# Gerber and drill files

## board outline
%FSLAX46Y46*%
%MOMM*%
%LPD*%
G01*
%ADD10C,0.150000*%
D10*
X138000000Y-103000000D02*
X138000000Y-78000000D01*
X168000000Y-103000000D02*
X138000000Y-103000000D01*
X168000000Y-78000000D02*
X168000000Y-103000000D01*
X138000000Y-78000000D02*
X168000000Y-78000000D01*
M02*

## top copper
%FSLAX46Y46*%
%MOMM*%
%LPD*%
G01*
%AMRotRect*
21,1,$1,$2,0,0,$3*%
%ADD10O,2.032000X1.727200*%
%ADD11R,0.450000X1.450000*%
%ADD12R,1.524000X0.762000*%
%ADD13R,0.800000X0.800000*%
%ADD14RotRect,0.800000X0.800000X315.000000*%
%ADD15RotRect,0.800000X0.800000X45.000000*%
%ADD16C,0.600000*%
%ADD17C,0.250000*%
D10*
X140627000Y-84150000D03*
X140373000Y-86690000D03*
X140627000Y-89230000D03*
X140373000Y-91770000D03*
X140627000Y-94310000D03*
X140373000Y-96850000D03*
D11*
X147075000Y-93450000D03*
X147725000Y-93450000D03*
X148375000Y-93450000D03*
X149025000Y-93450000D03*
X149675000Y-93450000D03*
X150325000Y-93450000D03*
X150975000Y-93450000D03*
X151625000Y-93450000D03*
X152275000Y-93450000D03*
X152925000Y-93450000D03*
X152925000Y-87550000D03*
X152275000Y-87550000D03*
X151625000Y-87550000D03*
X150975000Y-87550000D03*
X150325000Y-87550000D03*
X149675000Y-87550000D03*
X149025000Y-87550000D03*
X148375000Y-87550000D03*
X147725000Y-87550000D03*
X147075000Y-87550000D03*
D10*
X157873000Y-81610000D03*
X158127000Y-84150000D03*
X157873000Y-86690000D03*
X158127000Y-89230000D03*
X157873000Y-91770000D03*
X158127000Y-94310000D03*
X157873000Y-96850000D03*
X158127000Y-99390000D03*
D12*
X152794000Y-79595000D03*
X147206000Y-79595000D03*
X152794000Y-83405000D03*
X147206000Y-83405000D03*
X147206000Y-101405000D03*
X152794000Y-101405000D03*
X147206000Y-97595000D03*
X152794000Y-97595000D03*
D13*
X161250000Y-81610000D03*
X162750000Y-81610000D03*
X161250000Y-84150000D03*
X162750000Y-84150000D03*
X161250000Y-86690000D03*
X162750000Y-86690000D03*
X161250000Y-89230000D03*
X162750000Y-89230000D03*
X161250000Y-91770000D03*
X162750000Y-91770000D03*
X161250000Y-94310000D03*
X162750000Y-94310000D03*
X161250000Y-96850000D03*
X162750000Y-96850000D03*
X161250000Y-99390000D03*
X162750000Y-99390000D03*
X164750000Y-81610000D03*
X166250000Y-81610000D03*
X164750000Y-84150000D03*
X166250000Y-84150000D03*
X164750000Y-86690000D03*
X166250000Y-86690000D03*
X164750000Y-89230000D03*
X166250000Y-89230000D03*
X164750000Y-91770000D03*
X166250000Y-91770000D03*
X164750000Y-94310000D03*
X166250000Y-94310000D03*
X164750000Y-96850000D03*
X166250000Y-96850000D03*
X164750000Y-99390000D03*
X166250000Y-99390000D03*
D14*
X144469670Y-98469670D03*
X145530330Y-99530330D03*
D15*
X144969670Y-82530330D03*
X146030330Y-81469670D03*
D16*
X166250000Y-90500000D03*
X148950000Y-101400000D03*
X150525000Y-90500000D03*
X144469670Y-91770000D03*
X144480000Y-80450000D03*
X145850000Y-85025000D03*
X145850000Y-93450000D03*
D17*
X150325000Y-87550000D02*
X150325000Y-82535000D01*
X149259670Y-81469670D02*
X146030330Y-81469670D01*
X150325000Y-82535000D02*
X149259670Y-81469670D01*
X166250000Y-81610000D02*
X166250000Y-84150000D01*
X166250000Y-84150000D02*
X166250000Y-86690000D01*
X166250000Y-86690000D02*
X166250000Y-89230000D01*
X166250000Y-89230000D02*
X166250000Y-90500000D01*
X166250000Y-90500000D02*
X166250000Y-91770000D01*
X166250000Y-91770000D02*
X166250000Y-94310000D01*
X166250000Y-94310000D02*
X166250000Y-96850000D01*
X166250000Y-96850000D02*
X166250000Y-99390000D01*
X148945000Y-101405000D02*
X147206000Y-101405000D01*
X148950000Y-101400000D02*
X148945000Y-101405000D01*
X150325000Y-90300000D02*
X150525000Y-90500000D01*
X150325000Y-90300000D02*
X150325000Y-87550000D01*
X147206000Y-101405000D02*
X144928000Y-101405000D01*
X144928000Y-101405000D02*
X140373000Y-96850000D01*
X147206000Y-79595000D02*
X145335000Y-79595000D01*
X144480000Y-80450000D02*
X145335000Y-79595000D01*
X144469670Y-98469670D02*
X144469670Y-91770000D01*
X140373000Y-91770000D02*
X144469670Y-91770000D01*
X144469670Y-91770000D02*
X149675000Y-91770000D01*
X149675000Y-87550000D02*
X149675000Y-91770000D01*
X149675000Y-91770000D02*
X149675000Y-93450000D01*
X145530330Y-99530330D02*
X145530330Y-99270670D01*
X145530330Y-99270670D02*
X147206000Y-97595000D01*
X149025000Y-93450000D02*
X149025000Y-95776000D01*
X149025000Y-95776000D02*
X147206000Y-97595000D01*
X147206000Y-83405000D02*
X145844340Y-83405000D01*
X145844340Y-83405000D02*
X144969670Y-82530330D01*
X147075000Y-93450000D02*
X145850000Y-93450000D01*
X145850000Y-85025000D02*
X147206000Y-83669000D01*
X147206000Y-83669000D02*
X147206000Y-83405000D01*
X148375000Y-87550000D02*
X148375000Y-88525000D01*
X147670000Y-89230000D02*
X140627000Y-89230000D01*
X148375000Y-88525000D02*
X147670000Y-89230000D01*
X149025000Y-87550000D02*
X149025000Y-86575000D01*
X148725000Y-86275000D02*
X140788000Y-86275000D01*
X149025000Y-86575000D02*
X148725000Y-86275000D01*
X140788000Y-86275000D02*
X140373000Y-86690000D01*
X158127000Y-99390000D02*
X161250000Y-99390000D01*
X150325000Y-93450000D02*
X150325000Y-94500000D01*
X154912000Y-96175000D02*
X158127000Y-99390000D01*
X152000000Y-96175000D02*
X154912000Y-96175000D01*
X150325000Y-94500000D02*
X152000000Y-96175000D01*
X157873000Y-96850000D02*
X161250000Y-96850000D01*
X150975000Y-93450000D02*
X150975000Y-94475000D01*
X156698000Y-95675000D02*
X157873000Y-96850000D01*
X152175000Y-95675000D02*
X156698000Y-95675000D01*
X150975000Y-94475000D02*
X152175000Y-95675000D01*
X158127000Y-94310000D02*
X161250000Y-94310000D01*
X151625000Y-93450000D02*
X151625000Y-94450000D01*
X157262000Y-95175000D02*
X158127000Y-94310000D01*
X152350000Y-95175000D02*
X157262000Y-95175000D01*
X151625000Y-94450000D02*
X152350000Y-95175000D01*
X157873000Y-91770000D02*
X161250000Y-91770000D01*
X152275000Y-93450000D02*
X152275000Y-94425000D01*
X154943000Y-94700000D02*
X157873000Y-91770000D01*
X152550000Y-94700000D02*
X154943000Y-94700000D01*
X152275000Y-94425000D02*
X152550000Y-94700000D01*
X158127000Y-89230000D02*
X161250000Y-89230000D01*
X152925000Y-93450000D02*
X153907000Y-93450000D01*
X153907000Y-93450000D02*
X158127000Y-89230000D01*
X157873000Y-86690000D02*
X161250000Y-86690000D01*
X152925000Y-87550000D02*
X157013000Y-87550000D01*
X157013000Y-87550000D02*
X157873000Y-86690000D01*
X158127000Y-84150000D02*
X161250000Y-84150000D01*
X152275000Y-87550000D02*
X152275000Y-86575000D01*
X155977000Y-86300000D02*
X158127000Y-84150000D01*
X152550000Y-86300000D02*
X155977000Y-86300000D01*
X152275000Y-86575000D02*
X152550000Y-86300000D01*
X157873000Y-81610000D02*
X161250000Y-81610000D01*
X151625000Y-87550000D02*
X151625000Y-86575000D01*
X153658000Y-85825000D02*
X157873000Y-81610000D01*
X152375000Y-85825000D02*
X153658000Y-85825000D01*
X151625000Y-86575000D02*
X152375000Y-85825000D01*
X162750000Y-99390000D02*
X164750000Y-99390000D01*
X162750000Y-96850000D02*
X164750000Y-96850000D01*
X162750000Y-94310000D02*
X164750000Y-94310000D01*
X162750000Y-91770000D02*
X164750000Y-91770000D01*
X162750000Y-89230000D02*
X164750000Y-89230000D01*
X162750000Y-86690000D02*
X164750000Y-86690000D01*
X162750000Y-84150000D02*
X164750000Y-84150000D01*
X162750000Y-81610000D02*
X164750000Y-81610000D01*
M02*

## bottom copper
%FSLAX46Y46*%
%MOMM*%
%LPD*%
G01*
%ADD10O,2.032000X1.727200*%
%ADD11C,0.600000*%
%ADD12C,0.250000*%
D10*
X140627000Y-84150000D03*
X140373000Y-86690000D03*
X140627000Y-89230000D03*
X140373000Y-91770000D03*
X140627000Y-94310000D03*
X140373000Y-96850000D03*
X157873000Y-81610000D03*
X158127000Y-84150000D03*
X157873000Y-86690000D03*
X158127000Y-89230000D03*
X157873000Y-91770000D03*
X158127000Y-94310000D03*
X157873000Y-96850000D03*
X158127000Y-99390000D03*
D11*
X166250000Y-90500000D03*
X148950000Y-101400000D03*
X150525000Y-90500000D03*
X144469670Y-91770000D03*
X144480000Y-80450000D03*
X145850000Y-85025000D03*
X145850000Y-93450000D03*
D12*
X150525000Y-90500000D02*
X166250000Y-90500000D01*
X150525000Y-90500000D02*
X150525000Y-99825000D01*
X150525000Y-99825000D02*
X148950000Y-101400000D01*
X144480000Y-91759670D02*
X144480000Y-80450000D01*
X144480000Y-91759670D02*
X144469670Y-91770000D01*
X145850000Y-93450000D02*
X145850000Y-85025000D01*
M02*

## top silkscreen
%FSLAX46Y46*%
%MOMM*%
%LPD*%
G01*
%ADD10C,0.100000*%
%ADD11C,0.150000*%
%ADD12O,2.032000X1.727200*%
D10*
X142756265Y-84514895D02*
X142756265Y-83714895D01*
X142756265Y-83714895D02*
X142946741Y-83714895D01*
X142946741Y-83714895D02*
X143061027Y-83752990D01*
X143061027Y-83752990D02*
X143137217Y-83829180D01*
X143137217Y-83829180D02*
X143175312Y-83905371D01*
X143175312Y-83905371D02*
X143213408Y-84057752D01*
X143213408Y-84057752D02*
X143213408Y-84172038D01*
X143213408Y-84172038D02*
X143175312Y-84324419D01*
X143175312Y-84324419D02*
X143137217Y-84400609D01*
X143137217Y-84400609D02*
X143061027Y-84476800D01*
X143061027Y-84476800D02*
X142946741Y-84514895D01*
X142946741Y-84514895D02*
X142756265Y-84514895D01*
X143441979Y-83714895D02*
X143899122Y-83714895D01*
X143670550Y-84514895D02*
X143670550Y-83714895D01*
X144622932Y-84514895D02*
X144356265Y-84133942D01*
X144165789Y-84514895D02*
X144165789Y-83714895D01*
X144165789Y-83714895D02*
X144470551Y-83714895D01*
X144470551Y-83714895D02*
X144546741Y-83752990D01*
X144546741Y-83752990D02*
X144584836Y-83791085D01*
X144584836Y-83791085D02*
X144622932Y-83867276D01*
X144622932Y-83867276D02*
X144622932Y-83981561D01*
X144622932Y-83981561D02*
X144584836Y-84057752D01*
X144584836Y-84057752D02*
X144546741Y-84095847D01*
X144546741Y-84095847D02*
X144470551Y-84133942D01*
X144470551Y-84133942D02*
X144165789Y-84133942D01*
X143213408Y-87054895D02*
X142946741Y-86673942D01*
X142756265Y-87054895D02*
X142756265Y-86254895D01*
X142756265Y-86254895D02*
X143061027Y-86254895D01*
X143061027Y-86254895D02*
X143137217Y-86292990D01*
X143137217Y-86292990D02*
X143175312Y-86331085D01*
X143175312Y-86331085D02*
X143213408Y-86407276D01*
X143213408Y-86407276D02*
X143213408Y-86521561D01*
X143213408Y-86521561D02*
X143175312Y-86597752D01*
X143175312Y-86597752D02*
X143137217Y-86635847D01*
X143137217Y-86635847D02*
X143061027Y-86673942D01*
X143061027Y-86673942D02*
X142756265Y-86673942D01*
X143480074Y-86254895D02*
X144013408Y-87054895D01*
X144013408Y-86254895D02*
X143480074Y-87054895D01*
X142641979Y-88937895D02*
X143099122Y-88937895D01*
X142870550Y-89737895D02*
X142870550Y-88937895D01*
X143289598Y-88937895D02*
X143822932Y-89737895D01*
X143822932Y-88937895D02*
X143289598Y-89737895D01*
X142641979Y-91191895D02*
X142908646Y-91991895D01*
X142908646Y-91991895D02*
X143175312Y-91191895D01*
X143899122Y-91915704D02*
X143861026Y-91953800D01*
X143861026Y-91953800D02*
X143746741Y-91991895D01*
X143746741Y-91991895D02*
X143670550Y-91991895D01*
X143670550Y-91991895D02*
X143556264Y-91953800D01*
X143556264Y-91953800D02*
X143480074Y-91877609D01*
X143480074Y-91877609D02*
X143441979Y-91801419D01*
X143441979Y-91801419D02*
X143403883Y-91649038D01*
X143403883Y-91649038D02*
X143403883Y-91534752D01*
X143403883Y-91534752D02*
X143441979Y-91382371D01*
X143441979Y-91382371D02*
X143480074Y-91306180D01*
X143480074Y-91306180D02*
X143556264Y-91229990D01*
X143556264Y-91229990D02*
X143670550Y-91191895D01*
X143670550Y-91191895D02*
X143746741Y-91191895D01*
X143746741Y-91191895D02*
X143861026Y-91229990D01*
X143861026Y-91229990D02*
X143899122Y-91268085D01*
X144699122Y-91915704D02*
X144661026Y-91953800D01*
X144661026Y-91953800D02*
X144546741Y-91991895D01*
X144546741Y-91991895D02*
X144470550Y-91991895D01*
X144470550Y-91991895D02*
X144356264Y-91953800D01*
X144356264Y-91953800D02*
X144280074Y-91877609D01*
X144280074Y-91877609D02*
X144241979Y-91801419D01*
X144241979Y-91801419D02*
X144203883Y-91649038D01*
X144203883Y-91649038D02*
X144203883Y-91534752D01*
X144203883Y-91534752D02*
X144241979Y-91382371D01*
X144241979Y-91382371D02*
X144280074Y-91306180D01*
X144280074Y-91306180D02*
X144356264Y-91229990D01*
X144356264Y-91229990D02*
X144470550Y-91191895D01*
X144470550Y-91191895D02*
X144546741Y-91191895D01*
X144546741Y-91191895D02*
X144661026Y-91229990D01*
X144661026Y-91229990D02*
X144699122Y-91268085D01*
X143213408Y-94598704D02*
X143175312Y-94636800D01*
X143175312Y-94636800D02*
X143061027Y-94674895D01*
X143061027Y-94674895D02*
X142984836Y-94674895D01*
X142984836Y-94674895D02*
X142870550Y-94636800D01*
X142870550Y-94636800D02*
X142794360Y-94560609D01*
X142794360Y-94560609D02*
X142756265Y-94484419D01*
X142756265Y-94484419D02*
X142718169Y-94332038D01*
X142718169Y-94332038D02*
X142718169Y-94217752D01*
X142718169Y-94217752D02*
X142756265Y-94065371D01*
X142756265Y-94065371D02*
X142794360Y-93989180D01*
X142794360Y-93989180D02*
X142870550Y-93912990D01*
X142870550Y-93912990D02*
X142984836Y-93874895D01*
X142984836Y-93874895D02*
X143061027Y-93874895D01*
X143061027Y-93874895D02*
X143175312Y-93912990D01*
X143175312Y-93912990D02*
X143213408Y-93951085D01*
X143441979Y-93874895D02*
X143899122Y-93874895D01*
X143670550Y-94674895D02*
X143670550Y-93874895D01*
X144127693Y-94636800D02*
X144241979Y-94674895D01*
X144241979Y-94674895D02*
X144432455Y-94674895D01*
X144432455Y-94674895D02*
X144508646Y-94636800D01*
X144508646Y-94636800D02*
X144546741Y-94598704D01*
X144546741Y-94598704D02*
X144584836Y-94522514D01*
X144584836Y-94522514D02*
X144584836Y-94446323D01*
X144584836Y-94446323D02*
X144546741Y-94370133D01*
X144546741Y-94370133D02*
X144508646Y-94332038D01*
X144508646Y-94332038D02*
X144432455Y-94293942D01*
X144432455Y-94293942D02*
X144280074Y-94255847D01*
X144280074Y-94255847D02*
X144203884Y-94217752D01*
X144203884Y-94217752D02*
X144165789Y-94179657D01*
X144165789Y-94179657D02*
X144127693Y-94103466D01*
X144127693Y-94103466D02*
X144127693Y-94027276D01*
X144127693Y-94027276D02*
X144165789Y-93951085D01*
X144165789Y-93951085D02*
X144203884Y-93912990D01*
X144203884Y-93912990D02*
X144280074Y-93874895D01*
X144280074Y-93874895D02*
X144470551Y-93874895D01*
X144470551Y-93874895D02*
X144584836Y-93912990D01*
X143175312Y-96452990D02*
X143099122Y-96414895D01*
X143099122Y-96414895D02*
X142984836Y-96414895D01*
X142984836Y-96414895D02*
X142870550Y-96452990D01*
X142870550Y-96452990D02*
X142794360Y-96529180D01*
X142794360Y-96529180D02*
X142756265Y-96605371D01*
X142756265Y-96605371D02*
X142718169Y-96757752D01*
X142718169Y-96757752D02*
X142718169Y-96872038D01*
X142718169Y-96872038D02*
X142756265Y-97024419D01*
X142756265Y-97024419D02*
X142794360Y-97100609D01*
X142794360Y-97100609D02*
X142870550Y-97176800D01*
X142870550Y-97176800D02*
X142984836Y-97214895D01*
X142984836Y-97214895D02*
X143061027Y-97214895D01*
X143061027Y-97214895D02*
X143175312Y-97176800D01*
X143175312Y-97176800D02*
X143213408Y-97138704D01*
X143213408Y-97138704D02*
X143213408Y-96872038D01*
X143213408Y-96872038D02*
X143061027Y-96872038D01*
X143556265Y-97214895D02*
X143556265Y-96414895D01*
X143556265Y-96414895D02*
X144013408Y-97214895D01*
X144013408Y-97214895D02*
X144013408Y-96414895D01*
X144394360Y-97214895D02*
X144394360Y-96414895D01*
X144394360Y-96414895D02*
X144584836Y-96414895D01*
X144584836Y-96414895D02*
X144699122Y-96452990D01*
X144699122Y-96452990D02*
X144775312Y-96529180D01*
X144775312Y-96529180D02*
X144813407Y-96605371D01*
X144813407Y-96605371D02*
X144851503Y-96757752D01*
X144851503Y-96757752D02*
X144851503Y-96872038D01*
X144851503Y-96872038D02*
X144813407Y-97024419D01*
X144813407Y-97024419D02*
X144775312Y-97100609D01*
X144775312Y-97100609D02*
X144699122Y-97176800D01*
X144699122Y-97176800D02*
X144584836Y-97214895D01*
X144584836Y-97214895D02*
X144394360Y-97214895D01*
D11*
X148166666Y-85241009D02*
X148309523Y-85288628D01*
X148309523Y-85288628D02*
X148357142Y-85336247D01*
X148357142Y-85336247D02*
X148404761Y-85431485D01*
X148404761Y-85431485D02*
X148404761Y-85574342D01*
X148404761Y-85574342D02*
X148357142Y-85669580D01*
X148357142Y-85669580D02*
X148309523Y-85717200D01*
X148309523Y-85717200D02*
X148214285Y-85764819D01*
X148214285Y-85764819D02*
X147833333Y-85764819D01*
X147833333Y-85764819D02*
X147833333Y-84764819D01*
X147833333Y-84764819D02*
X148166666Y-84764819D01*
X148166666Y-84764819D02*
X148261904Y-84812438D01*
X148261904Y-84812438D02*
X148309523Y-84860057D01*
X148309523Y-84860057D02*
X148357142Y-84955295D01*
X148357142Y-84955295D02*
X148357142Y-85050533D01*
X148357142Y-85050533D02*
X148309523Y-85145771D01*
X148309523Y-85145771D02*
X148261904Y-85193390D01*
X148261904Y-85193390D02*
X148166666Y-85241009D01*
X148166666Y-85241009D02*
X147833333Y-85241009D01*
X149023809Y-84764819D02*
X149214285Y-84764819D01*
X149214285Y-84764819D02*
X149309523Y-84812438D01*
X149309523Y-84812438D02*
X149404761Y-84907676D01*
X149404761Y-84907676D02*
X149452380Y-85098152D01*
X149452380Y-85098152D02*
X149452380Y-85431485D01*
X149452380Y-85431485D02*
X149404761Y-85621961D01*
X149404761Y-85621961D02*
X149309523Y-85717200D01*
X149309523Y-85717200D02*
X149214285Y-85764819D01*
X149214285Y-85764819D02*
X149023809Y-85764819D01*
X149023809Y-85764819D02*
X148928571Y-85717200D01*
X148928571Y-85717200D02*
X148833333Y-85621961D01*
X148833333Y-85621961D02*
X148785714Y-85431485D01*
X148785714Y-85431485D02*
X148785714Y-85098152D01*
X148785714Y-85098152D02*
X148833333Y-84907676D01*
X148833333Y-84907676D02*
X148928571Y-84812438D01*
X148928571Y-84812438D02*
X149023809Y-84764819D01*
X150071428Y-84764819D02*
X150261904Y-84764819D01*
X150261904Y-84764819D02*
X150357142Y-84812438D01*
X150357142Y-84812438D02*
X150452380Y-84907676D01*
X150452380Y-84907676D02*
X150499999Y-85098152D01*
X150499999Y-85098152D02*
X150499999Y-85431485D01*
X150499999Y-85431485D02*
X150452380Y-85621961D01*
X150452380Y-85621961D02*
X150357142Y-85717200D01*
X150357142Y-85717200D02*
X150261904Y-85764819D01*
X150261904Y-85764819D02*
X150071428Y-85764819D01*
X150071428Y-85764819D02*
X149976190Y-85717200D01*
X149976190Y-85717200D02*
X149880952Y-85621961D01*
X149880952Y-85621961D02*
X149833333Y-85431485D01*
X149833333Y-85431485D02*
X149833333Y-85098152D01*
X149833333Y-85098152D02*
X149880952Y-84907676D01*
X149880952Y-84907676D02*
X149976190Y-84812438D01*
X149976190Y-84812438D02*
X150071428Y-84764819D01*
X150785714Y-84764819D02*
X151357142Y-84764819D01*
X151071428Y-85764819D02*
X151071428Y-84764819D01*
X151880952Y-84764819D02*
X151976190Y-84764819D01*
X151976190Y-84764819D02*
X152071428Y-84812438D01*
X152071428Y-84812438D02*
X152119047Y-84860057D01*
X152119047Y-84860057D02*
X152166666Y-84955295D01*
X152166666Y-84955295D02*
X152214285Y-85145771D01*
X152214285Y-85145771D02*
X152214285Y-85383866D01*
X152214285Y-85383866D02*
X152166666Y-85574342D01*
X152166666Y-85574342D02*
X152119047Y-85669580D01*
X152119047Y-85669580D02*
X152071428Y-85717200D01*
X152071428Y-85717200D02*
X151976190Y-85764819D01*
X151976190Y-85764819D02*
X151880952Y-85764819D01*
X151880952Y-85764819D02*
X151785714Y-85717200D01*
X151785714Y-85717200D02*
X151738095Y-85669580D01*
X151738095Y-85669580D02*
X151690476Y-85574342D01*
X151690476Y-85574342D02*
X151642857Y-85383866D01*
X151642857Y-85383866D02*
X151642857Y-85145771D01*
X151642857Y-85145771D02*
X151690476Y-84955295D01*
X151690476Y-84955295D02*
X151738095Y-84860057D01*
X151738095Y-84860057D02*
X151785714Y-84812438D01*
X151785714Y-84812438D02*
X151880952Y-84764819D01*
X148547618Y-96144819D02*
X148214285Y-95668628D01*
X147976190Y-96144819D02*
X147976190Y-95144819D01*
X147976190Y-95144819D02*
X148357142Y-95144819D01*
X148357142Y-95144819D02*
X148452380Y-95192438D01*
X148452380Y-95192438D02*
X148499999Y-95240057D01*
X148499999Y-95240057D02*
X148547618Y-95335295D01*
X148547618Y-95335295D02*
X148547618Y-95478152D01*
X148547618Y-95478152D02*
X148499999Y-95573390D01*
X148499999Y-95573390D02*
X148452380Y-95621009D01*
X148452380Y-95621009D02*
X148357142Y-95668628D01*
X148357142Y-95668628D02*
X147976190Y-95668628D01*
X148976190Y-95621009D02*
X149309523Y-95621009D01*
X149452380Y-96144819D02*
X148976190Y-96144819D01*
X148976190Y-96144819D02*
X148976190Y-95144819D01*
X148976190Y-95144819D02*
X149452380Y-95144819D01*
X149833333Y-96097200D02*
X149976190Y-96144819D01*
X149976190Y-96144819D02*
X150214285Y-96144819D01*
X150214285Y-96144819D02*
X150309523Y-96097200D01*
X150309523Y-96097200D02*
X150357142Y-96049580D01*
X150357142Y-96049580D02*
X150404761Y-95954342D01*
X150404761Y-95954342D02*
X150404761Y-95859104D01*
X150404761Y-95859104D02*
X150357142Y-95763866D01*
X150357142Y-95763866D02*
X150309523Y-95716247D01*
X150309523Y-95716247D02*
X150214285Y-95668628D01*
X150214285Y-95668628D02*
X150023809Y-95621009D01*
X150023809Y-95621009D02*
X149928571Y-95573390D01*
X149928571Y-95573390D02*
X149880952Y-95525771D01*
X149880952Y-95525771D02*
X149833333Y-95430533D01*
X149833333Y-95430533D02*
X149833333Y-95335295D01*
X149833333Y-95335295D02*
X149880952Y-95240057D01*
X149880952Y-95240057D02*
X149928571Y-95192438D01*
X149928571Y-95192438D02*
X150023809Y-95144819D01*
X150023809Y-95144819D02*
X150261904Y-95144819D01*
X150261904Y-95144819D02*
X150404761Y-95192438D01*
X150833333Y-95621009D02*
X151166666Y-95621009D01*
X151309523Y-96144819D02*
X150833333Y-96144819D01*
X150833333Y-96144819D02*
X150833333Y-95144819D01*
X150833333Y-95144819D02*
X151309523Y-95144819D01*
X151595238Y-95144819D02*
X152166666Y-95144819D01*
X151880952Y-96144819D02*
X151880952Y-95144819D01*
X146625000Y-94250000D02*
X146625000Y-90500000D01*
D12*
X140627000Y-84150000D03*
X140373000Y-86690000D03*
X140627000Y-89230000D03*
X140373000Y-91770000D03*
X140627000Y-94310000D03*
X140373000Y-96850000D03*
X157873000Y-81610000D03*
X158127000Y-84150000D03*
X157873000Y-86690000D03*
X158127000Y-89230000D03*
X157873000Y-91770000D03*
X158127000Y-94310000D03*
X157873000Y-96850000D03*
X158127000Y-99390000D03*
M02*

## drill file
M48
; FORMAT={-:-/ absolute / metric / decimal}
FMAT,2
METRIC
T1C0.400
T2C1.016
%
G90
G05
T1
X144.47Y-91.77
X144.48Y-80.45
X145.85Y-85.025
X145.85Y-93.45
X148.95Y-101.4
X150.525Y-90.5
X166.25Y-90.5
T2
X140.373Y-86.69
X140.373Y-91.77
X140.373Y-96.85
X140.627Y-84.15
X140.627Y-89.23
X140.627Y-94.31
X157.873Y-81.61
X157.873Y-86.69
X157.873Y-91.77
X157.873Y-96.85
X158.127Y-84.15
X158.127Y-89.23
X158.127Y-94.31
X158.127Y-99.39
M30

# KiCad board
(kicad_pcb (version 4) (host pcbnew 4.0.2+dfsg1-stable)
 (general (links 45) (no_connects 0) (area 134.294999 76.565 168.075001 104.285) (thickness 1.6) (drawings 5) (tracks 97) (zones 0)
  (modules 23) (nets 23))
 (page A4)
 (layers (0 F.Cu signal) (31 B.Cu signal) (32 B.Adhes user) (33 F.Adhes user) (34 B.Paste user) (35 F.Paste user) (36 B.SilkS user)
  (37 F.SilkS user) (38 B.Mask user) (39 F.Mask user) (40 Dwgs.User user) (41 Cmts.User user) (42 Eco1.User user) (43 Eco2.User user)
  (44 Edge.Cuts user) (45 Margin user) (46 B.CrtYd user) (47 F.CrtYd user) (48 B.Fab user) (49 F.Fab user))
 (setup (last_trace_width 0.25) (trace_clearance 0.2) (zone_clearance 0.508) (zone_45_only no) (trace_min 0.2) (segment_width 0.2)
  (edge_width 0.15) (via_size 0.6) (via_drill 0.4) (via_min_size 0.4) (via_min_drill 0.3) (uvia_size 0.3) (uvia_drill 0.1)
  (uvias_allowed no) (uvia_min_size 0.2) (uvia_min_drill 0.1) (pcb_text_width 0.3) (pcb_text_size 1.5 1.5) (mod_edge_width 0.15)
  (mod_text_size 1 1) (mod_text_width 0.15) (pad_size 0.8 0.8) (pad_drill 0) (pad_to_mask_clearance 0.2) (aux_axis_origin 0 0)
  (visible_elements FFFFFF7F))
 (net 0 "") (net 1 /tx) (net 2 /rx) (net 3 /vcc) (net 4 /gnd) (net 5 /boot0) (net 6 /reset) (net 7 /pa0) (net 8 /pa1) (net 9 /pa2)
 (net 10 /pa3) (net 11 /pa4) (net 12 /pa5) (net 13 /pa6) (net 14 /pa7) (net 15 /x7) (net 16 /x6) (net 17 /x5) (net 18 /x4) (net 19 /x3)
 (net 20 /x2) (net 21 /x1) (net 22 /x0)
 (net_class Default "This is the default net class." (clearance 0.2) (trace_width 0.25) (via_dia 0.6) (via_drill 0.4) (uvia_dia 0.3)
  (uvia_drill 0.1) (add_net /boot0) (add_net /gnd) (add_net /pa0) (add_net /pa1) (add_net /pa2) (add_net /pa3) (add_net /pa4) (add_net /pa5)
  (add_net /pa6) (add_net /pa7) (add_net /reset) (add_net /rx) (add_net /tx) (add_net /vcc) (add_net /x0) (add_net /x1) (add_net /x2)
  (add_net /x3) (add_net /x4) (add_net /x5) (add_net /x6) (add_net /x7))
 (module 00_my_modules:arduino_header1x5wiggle (layer F.Cu) (at 140.5 90.5)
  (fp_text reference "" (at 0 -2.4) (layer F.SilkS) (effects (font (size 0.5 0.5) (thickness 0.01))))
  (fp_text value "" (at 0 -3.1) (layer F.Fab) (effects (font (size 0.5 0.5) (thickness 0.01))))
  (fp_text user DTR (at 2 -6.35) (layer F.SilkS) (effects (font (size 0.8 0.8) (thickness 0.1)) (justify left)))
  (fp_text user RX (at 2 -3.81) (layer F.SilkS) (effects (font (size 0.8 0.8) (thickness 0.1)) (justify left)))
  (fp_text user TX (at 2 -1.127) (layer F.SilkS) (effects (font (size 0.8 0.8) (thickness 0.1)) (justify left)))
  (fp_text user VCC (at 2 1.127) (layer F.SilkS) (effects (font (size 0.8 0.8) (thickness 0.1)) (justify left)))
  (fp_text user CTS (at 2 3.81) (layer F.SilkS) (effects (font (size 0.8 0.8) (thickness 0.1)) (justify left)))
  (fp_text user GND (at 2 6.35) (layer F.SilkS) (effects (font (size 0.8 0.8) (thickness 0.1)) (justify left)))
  (pad DTR thru_hole oval (at 0.127 -6.35) (size 2.032 1.7272) (drill 1.016) (layers *.Cu *.Mask F.SilkS))
  (pad RX thru_hole oval (at -0.127 -3.81) (size 2.032 1.7272) (drill 1.016) (layers *.Cu *.Mask F.SilkS) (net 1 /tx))
  (pad TX thru_hole oval (at 0.127 -1.27) (size 2.032 1.7272) (drill 1.016) (layers *.Cu *.Mask F.SilkS) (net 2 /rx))
  (pad VCC thru_hole oval (at -0.127 1.27) (size 2.032 1.7272) (drill 1.016) (layers *.Cu *.Mask F.SilkS) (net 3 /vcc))
  (pad CTS thru_hole oval (at 0.127 3.81) (size 2.032 1.7272) (drill 1.016) (layers *.Cu *.Mask F.SilkS))
  (pad GND thru_hole oval (at -0.127 6.35) (size 2.032 1.7272) (drill 1.016) (layers *.Cu *.Mask F.SilkS) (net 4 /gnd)))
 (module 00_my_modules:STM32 (layer F.Cu) (at 150 90.5 90)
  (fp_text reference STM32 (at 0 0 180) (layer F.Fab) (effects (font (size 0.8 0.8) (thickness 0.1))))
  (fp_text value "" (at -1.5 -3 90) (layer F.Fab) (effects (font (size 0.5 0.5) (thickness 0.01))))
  (fp_line (start -3.75 -3.375) (end 0 -3.375) (layer F.SilkS) (width 0.15))
  (pad BOOT smd rect (at -2.95 -2.925 90) (size 1.45 0.45) (layers F.Cu F.Paste F.Mask) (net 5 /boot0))
  (pad 2 smd rect (at -2.95 -2.275 90) (size 1.45 0.45) (layers F.Cu F.Paste F.Mask))
  (pad 3 smd rect (at -2.95 -1.625 90) (size 1.45 0.45) (layers F.Cu F.Paste F.Mask))
  (pad NRST smd rect (at -2.95 -0.975 90) (size 1.45 0.45) (layers F.Cu F.Paste F.Mask) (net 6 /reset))
  (pad VCC smd rect (at -2.95 -0.325 90) (size 1.45 0.45) (layers F.Cu F.Paste F.Mask) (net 3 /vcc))
  (pad PA0 smd rect (at -2.95 0.325 90) (size 1.45 0.45) (layers F.Cu F.Paste F.Mask) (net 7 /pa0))
  (pad PA1 smd rect (at -2.95 0.975 90) (size 1.45 0.45) (layers F.Cu F.Paste F.Mask) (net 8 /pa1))
  (pad PA2 smd rect (at -2.95 1.625 90) (size 1.45 0.45) (layers F.Cu F.Paste F.Mask) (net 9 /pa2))
  (pad PA3 smd rect (at -2.95 2.275 90) (size 1.45 0.45) (layers F.Cu F.Paste F.Mask) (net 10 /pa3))
  (pad PA4 smd rect (at -2.95 2.925 90) (size 1.45 0.45) (layers F.Cu F.Paste F.Mask) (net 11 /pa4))
  (pad PA5 smd rect (at 2.95 2.925 90) (size 1.45 0.45) (layers F.Cu F.Paste F.Mask) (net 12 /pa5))
  (pad PA6 smd rect (at 2.95 2.275 90) (size 1.45 0.45) (layers F.Cu F.Paste F.Mask) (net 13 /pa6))
  (pad PA7 smd rect (at 2.95 1.625 90) (size 1.45 0.45) (layers F.Cu F.Paste F.Mask) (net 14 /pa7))
  (pad PB1 smd rect (at 2.95 0.975 90) (size 1.45 0.45) (layers F.Cu F.Paste F.Mask))
  (pad GND smd rect (at 2.95 0.325 90) (size 1.45 0.45) (layers F.Cu F.Paste F.Mask) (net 4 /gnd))
  (pad VCC smd rect (at 2.95 -0.325 90) (size 1.45 0.45) (layers F.Cu F.Paste F.Mask) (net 3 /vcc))
  (pad TX smd rect (at 2.95 -0.975 90) (size 1.45 0.45) (layers F.Cu F.Paste F.Mask) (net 1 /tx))
  (pad RX smd rect (at 2.95 -1.625 90) (size 1.45 0.45) (layers F.Cu F.Paste F.Mask) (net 2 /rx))
  (pad DIO smd rect (at 2.95 -2.275 90) (size 1.45 0.45) (layers F.Cu F.Paste F.Mask))
  (pad CLK smd rect (at 2.95 -2.925 90) (size 1.45 0.45) (layers F.Cu F.Paste F.Mask)))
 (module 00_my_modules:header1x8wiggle (layer F.Cu) (at 158 90.5)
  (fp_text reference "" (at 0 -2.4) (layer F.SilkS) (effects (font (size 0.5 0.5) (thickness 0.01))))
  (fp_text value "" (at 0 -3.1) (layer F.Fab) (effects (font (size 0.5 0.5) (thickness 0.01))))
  (pad 7 thru_hole oval (at -0.127 -8.89) (size 2.032 1.7272) (drill 1.016) (layers *.Cu *.Mask F.SilkS) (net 14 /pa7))
  (pad 6 thru_hole oval (at 0.127 -6.35) (size 2.032 1.7272) (drill 1.016) (layers *.Cu *.Mask F.SilkS) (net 13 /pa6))
  (pad 5 thru_hole oval (at -0.127 -3.81) (size 2.032 1.7272) (drill 1.016) (layers *.Cu *.Mask F.SilkS) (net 12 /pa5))
  (pad 4 thru_hole oval (at 0.127 -1.27) (size 2.032 1.7272) (drill 1.016) (layers *.Cu *.Mask F.SilkS) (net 11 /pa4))
  (pad 3 thru_hole oval (at -0.127 1.27) (size 2.032 1.7272) (drill 1.016) (layers *.Cu *.Mask F.SilkS) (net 10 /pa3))
  (pad 2 thru_hole oval (at 0.127 3.81) (size 2.032 1.7272) (drill 1.016) (layers *.Cu *.Mask F.SilkS) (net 9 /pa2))
  (pad 1 thru_hole oval (at -0.127 6.35) (size 2.032 1.7272) (drill 1.016) (layers *.Cu *.Mask F.SilkS) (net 8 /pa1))
  (pad 0 thru_hole oval (at 0.127 8.89) (size 2.032 1.7272) (drill 1.016) (layers *.Cu *.Mask F.SilkS) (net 7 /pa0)))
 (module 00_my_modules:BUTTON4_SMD (layer F.Cu) (at 150 81.5 180)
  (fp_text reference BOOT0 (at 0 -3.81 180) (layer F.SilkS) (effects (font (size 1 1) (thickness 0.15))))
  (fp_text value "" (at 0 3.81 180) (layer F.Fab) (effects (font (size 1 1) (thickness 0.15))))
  (pad 1 smd rect (at -2.794 1.905 180) (size 1.524 0.762) (layers F.Cu F.Paste F.Mask))
  (pad 2 smd rect (at 2.794 1.905 180) (size 1.524 0.762) (layers F.Cu F.Paste F.Mask) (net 3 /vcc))
  (pad 3 smd rect (at -2.794 -1.905 180) (size 1.524 0.762) (layers F.Cu F.Paste F.Mask))
  (pad 4 smd rect (at 2.794 -1.905 180) (size 1.524 0.762) (layers F.Cu F.Paste F.Mask) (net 5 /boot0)))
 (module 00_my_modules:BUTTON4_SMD (layer F.Cu) (at 150 99.5)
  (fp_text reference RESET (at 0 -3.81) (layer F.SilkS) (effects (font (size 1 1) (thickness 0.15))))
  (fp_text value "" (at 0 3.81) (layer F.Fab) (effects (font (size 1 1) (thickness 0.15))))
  (pad 1 smd rect (at -2.794 1.905) (size 1.524 0.762) (layers F.Cu F.Paste F.Mask) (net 4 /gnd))
  (pad 2 smd rect (at 2.794 1.905) (size 1.524 0.762) (layers F.Cu F.Paste F.Mask))
  (pad 3 smd rect (at -2.794 -1.905) (size 1.524 0.762) (layers F.Cu F.Paste F.Mask) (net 6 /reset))
  (pad 4 smd rect (at 2.794 -1.905) (size 1.524 0.762) (layers F.Cu F.Paste F.Mask)))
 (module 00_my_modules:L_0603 (layer F.Cu) (at 162 81.61)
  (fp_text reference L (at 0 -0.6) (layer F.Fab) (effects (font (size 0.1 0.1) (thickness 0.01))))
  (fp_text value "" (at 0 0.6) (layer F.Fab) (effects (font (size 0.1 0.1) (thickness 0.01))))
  (pad 1 smd rect (at -0.75 0) (size 0.8 0.8) (layers F.Cu F.Paste F.Mask) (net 14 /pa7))
  (pad 2 smd rect (at 0.75 0) (size 0.8 0.8) (layers F.Cu F.Paste F.Mask) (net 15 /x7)))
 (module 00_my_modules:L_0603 (layer F.Cu) (at 162 84.15)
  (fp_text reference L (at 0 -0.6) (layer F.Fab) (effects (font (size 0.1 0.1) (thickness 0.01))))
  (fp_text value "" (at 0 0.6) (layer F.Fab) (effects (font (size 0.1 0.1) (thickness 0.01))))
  (pad 1 smd rect (at -0.75 0) (size 0.8 0.8) (layers F.Cu F.Paste F.Mask) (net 13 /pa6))
  (pad 2 smd rect (at 0.75 0) (size 0.8 0.8) (layers F.Cu F.Paste F.Mask) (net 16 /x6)))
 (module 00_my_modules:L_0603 (layer F.Cu) (at 162 86.69)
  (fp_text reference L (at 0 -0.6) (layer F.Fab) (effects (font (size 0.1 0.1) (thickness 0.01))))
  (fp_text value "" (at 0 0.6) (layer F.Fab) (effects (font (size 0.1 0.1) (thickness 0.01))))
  (pad 1 smd rect (at -0.75 0) (size 0.8 0.8) (layers F.Cu F.Paste F.Mask) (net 12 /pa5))
  (pad 2 smd rect (at 0.75 0) (size 0.8 0.8) (layers F.Cu F.Paste F.Mask) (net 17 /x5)))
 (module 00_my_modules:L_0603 (layer F.Cu) (at 162 89.23)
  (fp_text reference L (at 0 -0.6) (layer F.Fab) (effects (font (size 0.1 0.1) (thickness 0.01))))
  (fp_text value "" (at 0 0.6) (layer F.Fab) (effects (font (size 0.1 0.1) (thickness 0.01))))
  (pad 1 smd rect (at -0.75 0) (size 0.8 0.8) (layers F.Cu F.Paste F.Mask) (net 11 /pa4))
  (pad 4 smd rect (at 0.75 0) (size 0.8 0.8) (layers F.Cu F.Paste F.Mask) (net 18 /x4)))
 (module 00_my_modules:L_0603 (layer F.Cu) (at 162 91.77)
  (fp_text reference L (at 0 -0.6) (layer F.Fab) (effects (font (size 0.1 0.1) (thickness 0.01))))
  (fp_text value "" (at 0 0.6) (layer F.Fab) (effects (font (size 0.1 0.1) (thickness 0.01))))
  (pad 1 smd rect (at -0.75 0) (size 0.8 0.8) (layers F.Cu F.Paste F.Mask) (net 10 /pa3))
  (pad 2 smd rect (at 0.75 0) (size 0.8 0.8) (layers F.Cu F.Paste F.Mask) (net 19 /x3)))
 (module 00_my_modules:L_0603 (layer F.Cu) (at 162 94.31)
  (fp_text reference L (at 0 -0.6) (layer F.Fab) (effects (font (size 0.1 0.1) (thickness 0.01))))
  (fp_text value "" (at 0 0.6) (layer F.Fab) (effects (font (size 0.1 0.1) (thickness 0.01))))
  (pad 1 smd rect (at -0.75 0) (size 0.8 0.8) (layers F.Cu F.Paste F.Mask) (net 9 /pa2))
  (pad 2 smd rect (at 0.75 0) (size 0.8 0.8) (layers F.Cu F.Paste F.Mask) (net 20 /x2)))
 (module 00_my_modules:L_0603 (layer F.Cu) (at 162 96.85)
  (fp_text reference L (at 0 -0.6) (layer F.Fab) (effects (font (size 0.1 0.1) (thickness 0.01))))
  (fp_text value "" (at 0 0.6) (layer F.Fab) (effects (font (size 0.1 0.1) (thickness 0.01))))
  (pad 1 smd rect (at -0.75 0) (size 0.8 0.8) (layers F.Cu F.Paste F.Mask) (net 8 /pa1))
  (pad 2 smd rect (at 0.75 0) (size 0.8 0.8) (layers F.Cu F.Paste F.Mask) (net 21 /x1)))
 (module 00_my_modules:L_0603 (layer F.Cu) (at 162 99.39)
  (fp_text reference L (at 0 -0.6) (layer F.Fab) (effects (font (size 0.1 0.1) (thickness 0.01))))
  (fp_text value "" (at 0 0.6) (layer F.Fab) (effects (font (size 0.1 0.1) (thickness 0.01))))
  (pad 1 smd rect (at -0.75 0) (size 0.8 0.8) (layers F.Cu F.Paste F.Mask) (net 7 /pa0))
  (pad 2 smd rect (at 0.75 0) (size 0.8 0.8) (layers F.Cu F.Paste F.Mask) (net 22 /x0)))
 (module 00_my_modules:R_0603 (layer F.Cu) (at 165.5 81.61)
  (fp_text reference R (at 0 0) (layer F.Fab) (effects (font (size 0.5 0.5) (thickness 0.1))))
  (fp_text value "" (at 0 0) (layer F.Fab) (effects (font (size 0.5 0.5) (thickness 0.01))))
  (pad 1 smd rect (at -0.75 0) (size 0.8 0.8) (layers F.Cu F.Paste F.Mask) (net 15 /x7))
  (pad 2 smd rect (at 0.75 0) (size 0.8 0.8) (layers F.Cu F.Paste F.Mask) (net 4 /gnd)))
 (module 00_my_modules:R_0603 (layer F.Cu) (at 165.5 84.15)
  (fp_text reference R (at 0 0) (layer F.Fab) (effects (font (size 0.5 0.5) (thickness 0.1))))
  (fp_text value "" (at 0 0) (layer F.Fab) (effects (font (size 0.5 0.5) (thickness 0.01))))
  (pad 1 smd rect (at -0.75 0) (size 0.8 0.8) (layers F.Cu F.Paste F.Mask) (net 16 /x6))
  (pad 2 smd rect (at 0.75 0) (size 0.8 0.8) (layers F.Cu F.Paste F.Mask) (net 4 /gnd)))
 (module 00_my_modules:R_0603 (layer F.Cu) (at 165.5 86.69)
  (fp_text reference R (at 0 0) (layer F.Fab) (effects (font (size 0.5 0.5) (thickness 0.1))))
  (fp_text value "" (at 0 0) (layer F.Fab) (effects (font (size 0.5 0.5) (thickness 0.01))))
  (pad 1 smd rect (at -0.75 0) (size 0.8 0.8) (layers F.Cu F.Paste F.Mask) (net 17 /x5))
  (pad 2 smd rect (at 0.75 0) (size 0.8 0.8) (layers F.Cu F.Paste F.Mask) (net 4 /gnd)))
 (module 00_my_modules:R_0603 (layer F.Cu) (at 165.5 89.23)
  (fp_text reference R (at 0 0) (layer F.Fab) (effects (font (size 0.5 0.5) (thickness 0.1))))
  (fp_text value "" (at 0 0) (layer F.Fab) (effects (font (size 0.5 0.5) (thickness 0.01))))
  (pad 1 smd rect (at -0.75 0) (size 0.8 0.8) (layers F.Cu F.Paste F.Mask) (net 18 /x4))
  (pad 2 smd rect (at 0.75 0) (size 0.8 0.8) (layers F.Cu F.Paste F.Mask) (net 4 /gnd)))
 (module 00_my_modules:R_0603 (layer F.Cu) (at 165.5 91.77)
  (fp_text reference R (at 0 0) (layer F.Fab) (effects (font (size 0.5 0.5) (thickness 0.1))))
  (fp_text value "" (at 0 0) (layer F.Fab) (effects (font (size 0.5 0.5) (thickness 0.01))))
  (pad 1 smd rect (at -0.75 0) (size 0.8 0.8) (layers F.Cu F.Paste F.Mask) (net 19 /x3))
  (pad 2 smd rect (at 0.75 0) (size 0.8 0.8) (layers F.Cu F.Paste F.Mask) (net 4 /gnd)))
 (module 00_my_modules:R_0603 (layer F.Cu) (at 165.5 94.31)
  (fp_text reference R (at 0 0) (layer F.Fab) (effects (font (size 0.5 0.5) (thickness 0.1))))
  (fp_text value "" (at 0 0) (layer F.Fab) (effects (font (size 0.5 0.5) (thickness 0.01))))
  (pad 1 smd rect (at -0.75 0) (size 0.8 0.8) (layers F.Cu F.Paste F.Mask) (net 20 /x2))
  (pad 2 smd rect (at 0.75 0) (size 0.8 0.8) (layers F.Cu F.Paste F.Mask) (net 4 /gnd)))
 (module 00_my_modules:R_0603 (layer F.Cu) (at 165.5 96.85)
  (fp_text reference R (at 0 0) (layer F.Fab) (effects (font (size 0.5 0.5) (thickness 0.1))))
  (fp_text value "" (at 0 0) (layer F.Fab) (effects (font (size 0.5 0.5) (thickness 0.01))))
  (pad 1 smd rect (at -0.75 0) (size 0.8 0.8) (layers F.Cu F.Paste F.Mask) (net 21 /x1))
  (pad 2 smd rect (at 0.75 0) (size 0.8 0.8) (layers F.Cu F.Paste F.Mask) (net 4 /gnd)))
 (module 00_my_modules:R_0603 (layer F.Cu) (at 165.5 99.39)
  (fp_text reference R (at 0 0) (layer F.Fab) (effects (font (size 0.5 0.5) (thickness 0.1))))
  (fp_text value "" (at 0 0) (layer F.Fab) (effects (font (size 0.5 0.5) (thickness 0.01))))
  (pad 1 smd rect (at -0.75 0) (size 0.8 0.8) (layers F.Cu F.Paste F.Mask) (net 22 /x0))
  (pad 2 smd rect (at 0.75 0) (size 0.8 0.8) (layers F.Cu F.Paste F.Mask) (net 4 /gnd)))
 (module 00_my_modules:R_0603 (layer F.Cu) (at 145 99 315)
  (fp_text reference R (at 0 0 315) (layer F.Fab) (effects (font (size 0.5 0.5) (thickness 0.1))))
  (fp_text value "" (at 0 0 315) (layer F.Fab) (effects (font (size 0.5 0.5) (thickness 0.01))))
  (pad 1 smd rect (at -0.75 0 315) (size 0.8 0.8) (layers F.Cu F.Paste F.Mask) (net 3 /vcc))
  (pad 2 smd rect (at 0.75 0 315) (size 0.8 0.8) (layers F.Cu F.Paste F.Mask) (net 6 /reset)))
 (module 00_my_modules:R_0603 (layer F.Cu) (at 145.5 82 45)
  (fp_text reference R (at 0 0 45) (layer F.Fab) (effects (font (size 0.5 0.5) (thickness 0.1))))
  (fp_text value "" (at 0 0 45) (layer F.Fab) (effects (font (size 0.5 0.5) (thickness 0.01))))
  (pad 1 smd rect (at -0.75 0 45) (size 0.8 0.8) (layers F.Cu F.Paste F.Mask) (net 5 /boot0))
  (pad 2 smd rect (at 0.75 0 45) (size 0.8 0.8) (layers F.Cu F.Paste F.Mask) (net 4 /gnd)))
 (gr_line (start 138 103) (end 138 78) (angle 90) (layer Edge.Cuts) (width 0.15))
 (gr_line (start 168 103) (end 138 103) (angle 90) (layer Edge.Cuts) (width 0.15))
 (gr_line (start 168 78) (end 168 103) (angle 90) (layer Edge.Cuts) (width 0.15))
 (gr_line (start 138 78) (end 168 78) (angle 90) (layer Edge.Cuts) (width 0.15))
 (segment (start 150.325 87.55) (end 150.325 82.535) (width 0.25) (layer F.Cu) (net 4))
 (segment (start 149.25967 81.46967) (end 146.03033 81.46967) (width 0.25) (layer F.Cu) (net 4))
 (segment (start 150.325 82.535) (end 149.25967 81.46967) (width 0.25) (layer F.Cu) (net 4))
 (segment (start 150.525 90.5) (end 166.25 90.5) (width 0.25) (layer B.Cu) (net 4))
 (via (at 166.25 90.5) (size 0.6) (drill 0.4) (layers F.Cu B.Cu) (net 4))
 (segment (start 166.25 81.61) (end 166.25 84.15) (width 0.25) (layer F.Cu) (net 4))
 (segment (start 166.25 84.15) (end 166.25 86.69) (width 0.25) (layer F.Cu) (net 4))
 (segment (start 166.25 86.69) (end 166.25 89.23) (width 0.25) (layer F.Cu) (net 4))
 (segment (start 166.25 89.23) (end 166.25 90.5) (width 0.25) (layer F.Cu) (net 4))
 (segment (start 166.25 90.5) (end 166.25 91.77) (width 0.25) (layer F.Cu) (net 4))
 (segment (start 166.25 91.77) (end 166.25 94.31) (width 0.25) (layer F.Cu) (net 4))
 (segment (start 166.25 94.31) (end 166.25 96.85) (width 0.25) (layer F.Cu) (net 4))
 (segment (start 166.25 96.85) (end 166.25 99.39) (width 0.25) (layer F.Cu) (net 4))
 (segment (start 150.525 90.5) (end 150.525 99.825) (width 0.25) (layer B.Cu) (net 4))
 (segment (start 148.945 101.405) (end 147.206 101.405) (width 0.25) (layer F.Cu) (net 4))
 (segment (start 148.95 101.4) (end 148.945 101.405) (width 0.25) (layer F.Cu) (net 4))
 (via (at 148.95 101.4) (size 0.6) (drill 0.4) (layers F.Cu B.Cu) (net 4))
 (segment (start 150.525 99.825) (end 148.95 101.4) (width 0.25) (layer B.Cu) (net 4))
 (segment (start 150.325 90.3) (end 150.525 90.5) (width 0.25) (layer F.Cu) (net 4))
 (via (at 150.525 90.5) (size 0.6) (drill 0.4) (layers F.Cu B.Cu) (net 4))
 (segment (start 150.325 90.3) (end 150.325 87.55) (width 0.25) (layer F.Cu) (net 4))
 (segment (start 147.206 101.405) (end 144.928 101.405) (width 0.25) (layer F.Cu) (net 4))
 (segment (start 144.928 101.405) (end 140.373 96.85) (width 0.25) (layer F.Cu) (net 4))
 (via (at 144.46967 91.77) (size 0.6) (drill 0.4) (layers F.Cu B.Cu) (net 3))
 (segment (start 147.206 79.595) (end 145.335 79.595) (width 0.25) (layer F.Cu) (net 3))
 (segment (start 144.48 80.45) (end 145.335 79.595) (width 0.25) (layer F.Cu) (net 3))
 (via (at 144.48 80.45) (size 0.6) (drill 0.4) (layers F.Cu B.Cu) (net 3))
 (segment (start 144.48 91.75967) (end 144.48 80.45) (width 0.25) (layer B.Cu) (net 3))
 (segment (start 144.48 91.75967) (end 144.46967 91.77) (width 0.25) (layer B.Cu) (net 3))
 (segment (start 144.46967 98.46967) (end 144.46967 91.77) (width 0.25) (layer F.Cu) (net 3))
 (segment (start 140.373 91.77) (end 144.46967 91.77) (width 0.25) (layer F.Cu) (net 3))
 (segment (start 144.46967 91.77) (end 149.675 91.77) (width 0.25) (layer F.Cu) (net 3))
 (segment (start 149.675 87.55) (end 149.675 91.77) (width 0.25) (layer F.Cu) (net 3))
 (segment (start 149.675 91.77) (end 149.675 93.45) (width 0.25) (layer F.Cu) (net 3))
 (segment (start 145.53033 99.53033) (end 145.53033 99.27067) (width 0.25) (layer F.Cu) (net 6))
 (segment (start 145.53033 99.27067) (end 147.206 97.595) (width 0.25) (layer F.Cu) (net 6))
 (segment (start 149.025 93.45) (end 149.025 95.776) (width 0.25) (layer F.Cu) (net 6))
 (segment (start 149.025 95.776) (end 147.206 97.595) (width 0.25) (layer F.Cu) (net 6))
 (segment (start 147.206 83.405) (end 145.84434 83.405) (width 0.25) (layer F.Cu) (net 5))
 (segment (start 145.84434 83.405) (end 144.96967 82.53033) (width 0.25) (layer F.Cu) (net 5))
 (segment (start 147.075 93.45) (end 145.85 93.45) (width 0.25) (layer F.Cu) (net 5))
 (segment (start 145.85 85.025) (end 147.206 83.669) (width 0.25) (layer F.Cu) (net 5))
 (via (at 145.85 85.025) (size 0.6) (drill 0.4) (layers F.Cu B.Cu) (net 5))
 (segment (start 145.85 93.45) (end 145.85 85.025) (width 0.25) (layer B.Cu) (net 5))
 (via (at 145.85 93.45) (size 0.6) (drill 0.4) (layers F.Cu B.Cu) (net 5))
 (segment (start 147.206 83.669) (end 147.206 83.405) (width 0.25) (layer F.Cu) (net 5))
 (segment (start 148.375 87.55) (end 148.375 88.525) (width 0.25) (layer F.Cu) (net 2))
 (segment (start 147.67 89.23) (end 140.627 89.23) (width 0.25) (layer F.Cu) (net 2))
 (segment (start 148.375 88.525) (end 147.67 89.23) (width 0.25) (layer F.Cu) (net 2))
 (segment (start 149.025 87.55) (end 149.025 86.575) (width 0.25) (layer F.Cu) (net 1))
 (segment (start 148.725 86.275) (end 140.788 86.275) (width 0.25) (layer F.Cu) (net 1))
 (segment (start 149.025 86.575) (end 148.725 86.275) (width 0.25) (layer F.Cu) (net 1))
 (segment (start 140.788 86.275) (end 140.373 86.69) (width 0.25) (layer F.Cu) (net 1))
 (segment (start 158.127 99.39) (end 161.25 99.39) (width 0.25) (layer F.Cu) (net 7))
 (segment (start 150.325 93.45) (end 150.325 94.5) (width 0.25) (layer F.Cu) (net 7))
 (segment (start 154.912 96.175) (end 158.127 99.39) (width 0.25) (layer F.Cu) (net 7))
 (segment (start 152 96.175) (end 154.912 96.175) (width 0.25) (layer F.Cu) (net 7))
 (segment (start 150.325 94.5) (end 152 96.175) (width 0.25) (layer F.Cu) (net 7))
 (segment (start 157.873 96.85) (end 161.25 96.85) (width 0.25) (layer F.Cu) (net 8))
 (segment (start 150.975 93.45) (end 150.975 94.475) (width 0.25) (layer F.Cu) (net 8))
 (segment (start 156.698 95.675) (end 157.873 96.85) (width 0.25) (layer F.Cu) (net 8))
 (segment (start 152.175 95.675) (end 156.698 95.675) (width 0.25) (layer F.Cu) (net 8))
 (segment (start 150.975 94.475) (end 152.175 95.675) (width 0.25) (layer F.Cu) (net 8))
 (segment (start 158.127 94.31) (end 161.25 94.31) (width 0.25) (layer F.Cu) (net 9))
 (segment (start 151.625 93.45) (end 151.625 94.45) (width 0.25) (layer F.Cu) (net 9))
 (segment (start 157.262 95.175) (end 158.127 94.31) (width 0.25) (layer F.Cu) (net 9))
 (segment (start 152.35 95.175) (end 157.262 95.175) (width 0.25) (layer F.Cu) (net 9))
 (segment (start 151.625 94.45) (end 152.35 95.175) (width 0.25) (layer F.Cu) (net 9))
 (segment (start 157.873 91.77) (end 161.25 91.77) (width 0.25) (layer F.Cu) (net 10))
 (segment (start 152.275 93.45) (end 152.275 94.425) (width 0.25) (layer F.Cu) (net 10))
 (segment (start 154.943 94.7) (end 157.873 91.77) (width 0.25) (layer F.Cu) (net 10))
 (segment (start 152.55 94.7) (end 154.943 94.7) (width 0.25) (layer F.Cu) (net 10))
 (segment (start 152.275 94.425) (end 152.55 94.7) (width 0.25) (layer F.Cu) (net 10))
 (segment (start 158.127 89.23) (end 161.25 89.23) (width 0.25) (layer F.Cu) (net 11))
 (segment (start 152.925 93.45) (end 153.907 93.45) (width 0.25) (layer F.Cu) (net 11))
 (segment (start 153.907 93.45) (end 158.127 89.23) (width 0.25) (layer F.Cu) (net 11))
 (segment (start 157.873 86.69) (end 161.25 86.69) (width 0.25) (layer F.Cu) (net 12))
 (segment (start 152.925 87.55) (end 157.013 87.55) (width 0.25) (layer F.Cu) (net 12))
 (segment (start 157.013 87.55) (end 157.873 86.69) (width 0.25) (layer F.Cu) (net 12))
 (segment (start 158.127 84.15) (end 161.25 84.15) (width 0.25) (layer F.Cu) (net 13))
 (segment (start 152.275 87.55) (end 152.275 86.575) (width 0.25) (layer F.Cu) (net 13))
 (segment (start 155.977 86.3) (end 158.127 84.15) (width 0.25) (layer F.Cu) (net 13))
 (segment (start 152.55 86.3) (end 155.977 86.3) (width 0.25) (layer F.Cu) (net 13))
 (segment (start 152.275 86.575) (end 152.55 86.3) (width 0.25) (layer F.Cu) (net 13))
 (segment (start 157.873 81.61) (end 161.25 81.61) (width 0.25) (layer F.Cu) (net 14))
 (segment (start 151.625 87.55) (end 151.625 86.575) (width 0.25) (layer F.Cu) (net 14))
 (segment (start 153.658 85.825) (end 157.873 81.61) (width 0.25) (layer F.Cu) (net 14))
 (segment (start 152.375 85.825) (end 153.658 85.825) (width 0.25) (layer F.Cu) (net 14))
 (segment (start 151.625 86.575) (end 152.375 85.825) (width 0.25) (layer F.Cu) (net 14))
 (segment (start 162.75 99.39) (end 164.75 99.39) (width 0.25) (layer F.Cu) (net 22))
 (segment (start 162.75 96.85) (end 164.75 96.85) (width 0.25) (layer F.Cu) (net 21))
 (segment (start 162.75 94.31) (end 164.75 94.31) (width 0.25) (layer F.Cu) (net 20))
 (segment (start 162.75 91.77) (end 164.75 91.77) (width 0.25) (layer F.Cu) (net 19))
 (segment (start 162.75 89.23) (end 164.75 89.23) (width 0.25) (layer F.Cu) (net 18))
 (segment (start 162.75 86.69) (end 164.75 86.69) (width 0.25) (layer F.Cu) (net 17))
 (segment (start 162.75 84.15) (end 164.75 84.15) (width 0.25) (layer F.Cu) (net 16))
 (segment (start 162.75 81.61) (end 164.75 81.61) (width 0.25) (layer F.Cu) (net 15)))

